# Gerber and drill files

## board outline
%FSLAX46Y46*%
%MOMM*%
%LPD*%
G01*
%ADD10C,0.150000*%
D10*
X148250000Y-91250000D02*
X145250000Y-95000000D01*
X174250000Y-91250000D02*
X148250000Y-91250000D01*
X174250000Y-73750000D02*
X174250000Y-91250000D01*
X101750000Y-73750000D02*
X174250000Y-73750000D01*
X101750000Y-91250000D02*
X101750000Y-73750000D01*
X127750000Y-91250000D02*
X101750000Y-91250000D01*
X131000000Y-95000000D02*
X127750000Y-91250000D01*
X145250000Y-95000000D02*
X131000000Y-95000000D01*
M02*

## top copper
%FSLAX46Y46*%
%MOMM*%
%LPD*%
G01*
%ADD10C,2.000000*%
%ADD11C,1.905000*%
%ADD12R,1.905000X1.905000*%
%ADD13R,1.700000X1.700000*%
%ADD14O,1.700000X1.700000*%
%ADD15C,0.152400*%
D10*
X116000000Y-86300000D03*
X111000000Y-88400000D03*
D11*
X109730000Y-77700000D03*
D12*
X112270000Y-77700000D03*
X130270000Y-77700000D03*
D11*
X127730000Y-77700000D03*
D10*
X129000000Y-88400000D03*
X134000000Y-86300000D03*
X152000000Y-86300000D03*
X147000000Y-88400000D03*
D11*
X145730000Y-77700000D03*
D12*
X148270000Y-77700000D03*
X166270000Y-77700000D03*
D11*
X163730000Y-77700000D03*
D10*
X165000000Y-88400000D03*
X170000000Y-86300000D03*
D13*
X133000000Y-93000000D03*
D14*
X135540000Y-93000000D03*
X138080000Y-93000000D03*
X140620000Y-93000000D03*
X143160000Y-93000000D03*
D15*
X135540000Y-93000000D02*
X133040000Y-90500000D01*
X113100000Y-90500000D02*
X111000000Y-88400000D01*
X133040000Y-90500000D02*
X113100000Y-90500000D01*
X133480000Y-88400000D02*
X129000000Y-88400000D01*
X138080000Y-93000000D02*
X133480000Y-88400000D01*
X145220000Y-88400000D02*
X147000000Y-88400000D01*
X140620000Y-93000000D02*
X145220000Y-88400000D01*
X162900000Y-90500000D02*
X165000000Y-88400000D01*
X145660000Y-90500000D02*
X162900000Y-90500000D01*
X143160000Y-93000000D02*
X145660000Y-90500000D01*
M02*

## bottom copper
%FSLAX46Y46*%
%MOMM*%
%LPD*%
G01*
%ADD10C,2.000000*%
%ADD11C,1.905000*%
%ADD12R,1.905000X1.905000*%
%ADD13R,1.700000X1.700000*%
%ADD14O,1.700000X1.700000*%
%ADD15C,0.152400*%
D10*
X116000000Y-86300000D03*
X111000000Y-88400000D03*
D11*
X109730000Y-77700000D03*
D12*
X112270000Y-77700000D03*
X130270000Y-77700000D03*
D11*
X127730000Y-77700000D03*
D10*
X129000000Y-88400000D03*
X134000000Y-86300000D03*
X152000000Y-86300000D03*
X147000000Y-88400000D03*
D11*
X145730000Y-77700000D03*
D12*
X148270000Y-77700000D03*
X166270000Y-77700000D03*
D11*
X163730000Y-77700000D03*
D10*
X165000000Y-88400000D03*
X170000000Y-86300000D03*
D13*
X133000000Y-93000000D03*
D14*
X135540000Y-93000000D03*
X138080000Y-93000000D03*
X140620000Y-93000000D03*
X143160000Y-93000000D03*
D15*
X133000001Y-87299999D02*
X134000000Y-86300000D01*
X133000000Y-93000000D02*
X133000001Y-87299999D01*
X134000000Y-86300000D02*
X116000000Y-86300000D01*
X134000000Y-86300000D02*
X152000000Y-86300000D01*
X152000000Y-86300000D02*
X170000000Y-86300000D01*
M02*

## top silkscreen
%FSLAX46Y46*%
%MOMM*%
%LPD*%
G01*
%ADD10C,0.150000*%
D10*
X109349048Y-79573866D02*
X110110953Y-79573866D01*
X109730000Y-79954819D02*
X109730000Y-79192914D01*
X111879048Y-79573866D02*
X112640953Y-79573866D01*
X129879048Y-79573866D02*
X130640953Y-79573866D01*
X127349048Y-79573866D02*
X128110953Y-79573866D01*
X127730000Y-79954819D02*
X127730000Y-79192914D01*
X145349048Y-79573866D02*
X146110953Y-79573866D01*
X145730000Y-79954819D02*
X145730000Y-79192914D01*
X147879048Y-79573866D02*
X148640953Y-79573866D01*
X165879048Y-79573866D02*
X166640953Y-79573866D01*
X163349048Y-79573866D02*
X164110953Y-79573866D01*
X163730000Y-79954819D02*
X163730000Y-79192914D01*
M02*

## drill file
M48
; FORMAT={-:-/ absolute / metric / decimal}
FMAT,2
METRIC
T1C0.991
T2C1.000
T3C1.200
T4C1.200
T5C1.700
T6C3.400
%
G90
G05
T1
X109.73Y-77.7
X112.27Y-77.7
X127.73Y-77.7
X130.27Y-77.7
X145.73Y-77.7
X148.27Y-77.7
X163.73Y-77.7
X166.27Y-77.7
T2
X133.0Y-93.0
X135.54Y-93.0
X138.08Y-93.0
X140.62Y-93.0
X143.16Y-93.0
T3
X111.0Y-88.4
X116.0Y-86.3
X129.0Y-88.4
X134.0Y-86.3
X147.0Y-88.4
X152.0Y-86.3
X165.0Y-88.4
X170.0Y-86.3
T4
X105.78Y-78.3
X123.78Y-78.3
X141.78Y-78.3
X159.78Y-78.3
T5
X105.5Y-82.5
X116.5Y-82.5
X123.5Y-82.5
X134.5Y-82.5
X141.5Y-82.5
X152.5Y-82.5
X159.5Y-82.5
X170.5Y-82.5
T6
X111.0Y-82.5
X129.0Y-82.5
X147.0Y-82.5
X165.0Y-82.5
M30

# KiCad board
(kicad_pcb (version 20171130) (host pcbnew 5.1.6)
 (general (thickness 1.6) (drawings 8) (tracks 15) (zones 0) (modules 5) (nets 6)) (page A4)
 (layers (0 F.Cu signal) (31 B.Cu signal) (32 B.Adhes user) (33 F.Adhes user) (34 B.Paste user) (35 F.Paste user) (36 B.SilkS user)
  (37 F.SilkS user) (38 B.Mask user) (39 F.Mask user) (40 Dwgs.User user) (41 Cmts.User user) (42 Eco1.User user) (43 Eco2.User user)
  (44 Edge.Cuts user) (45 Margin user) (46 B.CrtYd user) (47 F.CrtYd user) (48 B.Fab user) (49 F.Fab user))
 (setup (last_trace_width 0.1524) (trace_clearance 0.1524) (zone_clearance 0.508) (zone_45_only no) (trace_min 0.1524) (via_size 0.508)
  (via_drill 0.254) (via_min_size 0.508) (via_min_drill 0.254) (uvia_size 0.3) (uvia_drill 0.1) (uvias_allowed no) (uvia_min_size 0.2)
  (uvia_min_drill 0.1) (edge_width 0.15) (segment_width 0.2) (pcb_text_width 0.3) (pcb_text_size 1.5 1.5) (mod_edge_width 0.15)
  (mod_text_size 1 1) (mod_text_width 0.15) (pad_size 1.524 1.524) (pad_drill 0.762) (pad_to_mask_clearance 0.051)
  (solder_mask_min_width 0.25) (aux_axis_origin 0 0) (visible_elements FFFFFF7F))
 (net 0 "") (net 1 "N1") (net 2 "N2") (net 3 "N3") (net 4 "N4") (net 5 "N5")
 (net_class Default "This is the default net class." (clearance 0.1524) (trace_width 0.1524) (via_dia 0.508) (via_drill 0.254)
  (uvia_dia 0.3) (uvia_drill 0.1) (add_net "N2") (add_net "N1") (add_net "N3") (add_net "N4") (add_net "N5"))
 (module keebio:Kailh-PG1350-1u (layer B.Cu) (at 111 82.5 180)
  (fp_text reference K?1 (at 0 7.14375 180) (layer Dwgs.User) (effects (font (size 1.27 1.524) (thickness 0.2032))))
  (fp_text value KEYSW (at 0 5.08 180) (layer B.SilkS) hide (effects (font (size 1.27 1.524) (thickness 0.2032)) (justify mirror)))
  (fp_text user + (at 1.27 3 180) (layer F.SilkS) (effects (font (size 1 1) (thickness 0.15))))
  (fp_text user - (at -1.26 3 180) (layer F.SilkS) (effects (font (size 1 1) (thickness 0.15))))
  (pad "" np_thru_hole circle (at 5.5 0) (size 1.7 1.7) (drill 1.7) (layers *.Cu))
  (pad "" np_thru_hole circle (at -5.5 0) (size 1.7 1.7) (drill 1.7) (layers *.Cu))
  (pad 2 thru_hole circle (at -5 -3.8 138.1) (size 2 2) (drill 1.2) (layers *.Cu *.Mask) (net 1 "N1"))
  (pad 1 thru_hole circle (at 0 -5.9) (size 2 2) (drill 1.2) (layers *.Cu *.Mask) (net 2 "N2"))
  (pad 3 thru_hole circle (at 1.27 4.8) (size 1.905 1.905) (drill 0.9906) (layers *.Cu *.Mask))
  (pad 4 thru_hole rect (at -1.27 4.8) (size 1.905 1.905) (drill 0.9906) (layers *.Cu *.Mask))
  (pad "" np_thru_hole circle (at 0 0) (size 3.4 3.4) (drill 3.4) (layers *.Cu))
  (pad "" np_thru_hole circle (at 5.22 4.2) (size 1.2 1.2) (drill 1.2) (layers *.Cu)))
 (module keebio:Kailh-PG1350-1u (layer B.Cu) (at 129 82.5 180)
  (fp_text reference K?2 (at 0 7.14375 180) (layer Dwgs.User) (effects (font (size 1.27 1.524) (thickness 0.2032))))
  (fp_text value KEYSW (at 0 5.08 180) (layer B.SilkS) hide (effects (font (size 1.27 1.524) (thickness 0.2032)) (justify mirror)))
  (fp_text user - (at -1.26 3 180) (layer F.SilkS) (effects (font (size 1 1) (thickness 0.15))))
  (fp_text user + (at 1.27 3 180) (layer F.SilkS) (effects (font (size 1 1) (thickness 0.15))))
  (pad "" np_thru_hole circle (at 5.22 4.2) (size 1.2 1.2) (drill 1.2) (layers *.Cu))
  (pad "" np_thru_hole circle (at 0 0) (size 3.4 3.4) (drill 3.4) (layers *.Cu))
  (pad 4 thru_hole rect (at -1.27 4.8) (size 1.905 1.905) (drill 0.9906) (layers *.Cu *.Mask))
  (pad 3 thru_hole circle (at 1.27 4.8) (size 1.905 1.905) (drill 0.9906) (layers *.Cu *.Mask))
  (pad 1 thru_hole circle (at 0 -5.9) (size 2 2) (drill 1.2) (layers *.Cu *.Mask) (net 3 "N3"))
  (pad 2 thru_hole circle (at -5 -3.8 138.1) (size 2 2) (drill 1.2) (layers *.Cu *.Mask) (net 1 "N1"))
  (pad "" np_thru_hole circle (at -5.5 0) (size 1.7 1.7) (drill 1.7) (layers *.Cu))
  (pad "" np_thru_hole circle (at 5.5 0) (size 1.7 1.7) (drill 1.7) (layers *.Cu)))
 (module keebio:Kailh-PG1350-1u (layer B.Cu) (at 147 82.5 180)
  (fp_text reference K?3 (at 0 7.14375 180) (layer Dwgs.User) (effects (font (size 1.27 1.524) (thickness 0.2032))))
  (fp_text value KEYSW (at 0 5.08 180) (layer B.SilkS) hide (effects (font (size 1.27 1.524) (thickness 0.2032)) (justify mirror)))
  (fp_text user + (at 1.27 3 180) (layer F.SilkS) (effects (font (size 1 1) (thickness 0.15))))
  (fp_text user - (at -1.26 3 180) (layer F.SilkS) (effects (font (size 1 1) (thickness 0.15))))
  (pad "" np_thru_hole circle (at 5.5 0) (size 1.7 1.7) (drill 1.7) (layers *.Cu))
  (pad "" np_thru_hole circle (at -5.5 0) (size 1.7 1.7) (drill 1.7) (layers *.Cu))
  (pad 2 thru_hole circle (at -5 -3.8 138.1) (size 2 2) (drill 1.2) (layers *.Cu *.Mask) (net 1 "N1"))
  (pad 1 thru_hole circle (at 0 -5.9) (size 2 2) (drill 1.2) (layers *.Cu *.Mask) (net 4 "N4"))
  (pad 3 thru_hole circle (at 1.27 4.8) (size 1.905 1.905) (drill 0.9906) (layers *.Cu *.Mask))
  (pad 4 thru_hole rect (at -1.27 4.8) (size 1.905 1.905) (drill 0.9906) (layers *.Cu *.Mask))
  (pad "" np_thru_hole circle (at 0 0) (size 3.4 3.4) (drill 3.4) (layers *.Cu))
  (pad "" np_thru_hole circle (at 5.22 4.2) (size 1.2 1.2) (drill 1.2) (layers *.Cu)))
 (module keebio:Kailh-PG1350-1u (layer B.Cu) (at 165 82.5 180)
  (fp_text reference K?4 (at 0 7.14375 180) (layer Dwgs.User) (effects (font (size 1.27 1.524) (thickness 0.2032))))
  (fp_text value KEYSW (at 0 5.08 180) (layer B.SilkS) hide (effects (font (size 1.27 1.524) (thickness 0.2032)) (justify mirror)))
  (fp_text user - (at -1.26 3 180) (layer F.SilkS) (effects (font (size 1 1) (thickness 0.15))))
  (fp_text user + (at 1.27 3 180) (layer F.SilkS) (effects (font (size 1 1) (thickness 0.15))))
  (pad "" np_thru_hole circle (at 5.22 4.2) (size 1.2 1.2) (drill 1.2) (layers *.Cu))
  (pad "" np_thru_hole circle (at 0 0) (size 3.4 3.4) (drill 3.4) (layers *.Cu))
  (pad 4 thru_hole rect (at -1.27 4.8) (size 1.905 1.905) (drill 0.9906) (layers *.Cu *.Mask))
  (pad 3 thru_hole circle (at 1.27 4.8) (size 1.905 1.905) (drill 0.9906) (layers *.Cu *.Mask))
  (pad 1 thru_hole circle (at 0 -5.9) (size 2 2) (drill 1.2) (layers *.Cu *.Mask) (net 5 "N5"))
  (pad 2 thru_hole circle (at -5 -3.8 138.1) (size 2 2) (drill 1.2) (layers *.Cu *.Mask) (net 1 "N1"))
  (pad "" np_thru_hole circle (at -5.5 0) (size 1.7 1.7) (drill 1.7) (layers *.Cu))
  (pad "" np_thru_hole circle (at 5.5 0) (size 1.7 1.7) (drill 1.7) (layers *.Cu)))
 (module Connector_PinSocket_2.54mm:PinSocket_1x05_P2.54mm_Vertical (layer B.Cu) (at 133 93 270)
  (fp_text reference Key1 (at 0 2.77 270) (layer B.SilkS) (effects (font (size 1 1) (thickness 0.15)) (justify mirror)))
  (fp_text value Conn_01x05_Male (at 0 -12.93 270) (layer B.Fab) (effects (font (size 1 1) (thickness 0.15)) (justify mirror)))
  (pad 1 thru_hole rect (at 0 0 270) (size 1.7 1.7) (drill 1) (layers *.Cu *.Mask) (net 1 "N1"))
  (pad 2 thru_hole oval (at 0 -2.54 270) (size 1.7 1.7) (drill 1) (layers *.Cu *.Mask) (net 2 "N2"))
  (pad 3 thru_hole oval (at 0 -5.08 270) (size 1.7 1.7) (drill 1) (layers *.Cu *.Mask) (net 3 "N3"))
  (pad 4 thru_hole oval (at 0 -7.62 270) (size 1.7 1.7) (drill 1) (layers *.Cu *.Mask) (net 4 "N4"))
  (pad 5 thru_hole oval (at 0 -10.16 270) (size 1.7 1.7) (drill 1) (layers *.Cu *.Mask) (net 5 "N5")))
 (gr_line (start 148.25 91.25) (end 145.25 95) (layer Edge.Cuts) (width 0.15))
 (gr_line (start 174.25 91.25) (end 148.25 91.25) (layer Edge.Cuts) (width 0.15))
 (gr_line (start 174.25 73.75) (end 174.25 91.25) (layer Edge.Cuts) (width 0.15))
 (gr_line (start 101.75 73.75) (end 174.25 73.75) (layer Edge.Cuts) (width 0.15))
 (gr_line (start 101.75 91.25) (end 101.75 73.75) (layer Edge.Cuts) (width 0.15))
 (gr_line (start 127.75 91.25) (end 101.75 91.25) (layer Edge.Cuts) (width 0.15))
 (gr_line (start 131 95) (end 127.75 91.25) (layer Edge.Cuts) (width 0.15))
 (gr_line (start 145.25 95) (end 131 95) (layer Edge.Cuts) (width 0.15))
 (segment (start 133.000001 87.299999) (end 134 86.3) (width 0.1524) (layer B.Cu) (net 1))
 (segment (start 133 93) (end 133.000001 87.299999) (width 0.1524) (layer B.Cu) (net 1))
 (segment (start 134 86.3) (end 116 86.3) (width 0.1524) (layer B.Cu) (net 1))
 (segment (start 134 86.3) (end 152 86.3) (width 0.1524) (layer B.Cu) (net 1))
 (segment (start 152 86.3) (end 170 86.3) (width 0.1524) (layer B.Cu) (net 1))
 (segment (start 135.54 93) (end 133.04 90.5) (width 0.1524) (layer F.Cu) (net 2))
 (segment (start 113.1 90.5) (end 111 88.4) (width 0.1524) (layer F.Cu) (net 2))
 (segment (start 133.04 90.5) (end 113.1 90.5) (width 0.1524) (layer F.Cu) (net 2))
 (segment (start 133.48 88.4) (end 129 88.4) (width 0.1524) (layer F.Cu) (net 3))
 (segment (start 138.08 93) (end 133.48 88.4) (width 0.1524) (layer F.Cu) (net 3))
 (segment (start 145.22 88.4) (end 147 88.4) (width 0.1524) (layer F.Cu) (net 4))
 (segment (start 140.62 93) (end 145.22 88.4) (width 0.1524) (layer F.Cu) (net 4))
 (segment (start 162.9 90.5) (end 165 88.4) (width 0.1524) (layer F.Cu) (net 5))
 (segment (start 145.66 90.5) (end 162.9 90.5) (width 0.1524) (layer F.Cu) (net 5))
 (segment (start 143.16 93) (end 145.66 90.5) (width 0.1524) (layer F.Cu) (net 5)))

